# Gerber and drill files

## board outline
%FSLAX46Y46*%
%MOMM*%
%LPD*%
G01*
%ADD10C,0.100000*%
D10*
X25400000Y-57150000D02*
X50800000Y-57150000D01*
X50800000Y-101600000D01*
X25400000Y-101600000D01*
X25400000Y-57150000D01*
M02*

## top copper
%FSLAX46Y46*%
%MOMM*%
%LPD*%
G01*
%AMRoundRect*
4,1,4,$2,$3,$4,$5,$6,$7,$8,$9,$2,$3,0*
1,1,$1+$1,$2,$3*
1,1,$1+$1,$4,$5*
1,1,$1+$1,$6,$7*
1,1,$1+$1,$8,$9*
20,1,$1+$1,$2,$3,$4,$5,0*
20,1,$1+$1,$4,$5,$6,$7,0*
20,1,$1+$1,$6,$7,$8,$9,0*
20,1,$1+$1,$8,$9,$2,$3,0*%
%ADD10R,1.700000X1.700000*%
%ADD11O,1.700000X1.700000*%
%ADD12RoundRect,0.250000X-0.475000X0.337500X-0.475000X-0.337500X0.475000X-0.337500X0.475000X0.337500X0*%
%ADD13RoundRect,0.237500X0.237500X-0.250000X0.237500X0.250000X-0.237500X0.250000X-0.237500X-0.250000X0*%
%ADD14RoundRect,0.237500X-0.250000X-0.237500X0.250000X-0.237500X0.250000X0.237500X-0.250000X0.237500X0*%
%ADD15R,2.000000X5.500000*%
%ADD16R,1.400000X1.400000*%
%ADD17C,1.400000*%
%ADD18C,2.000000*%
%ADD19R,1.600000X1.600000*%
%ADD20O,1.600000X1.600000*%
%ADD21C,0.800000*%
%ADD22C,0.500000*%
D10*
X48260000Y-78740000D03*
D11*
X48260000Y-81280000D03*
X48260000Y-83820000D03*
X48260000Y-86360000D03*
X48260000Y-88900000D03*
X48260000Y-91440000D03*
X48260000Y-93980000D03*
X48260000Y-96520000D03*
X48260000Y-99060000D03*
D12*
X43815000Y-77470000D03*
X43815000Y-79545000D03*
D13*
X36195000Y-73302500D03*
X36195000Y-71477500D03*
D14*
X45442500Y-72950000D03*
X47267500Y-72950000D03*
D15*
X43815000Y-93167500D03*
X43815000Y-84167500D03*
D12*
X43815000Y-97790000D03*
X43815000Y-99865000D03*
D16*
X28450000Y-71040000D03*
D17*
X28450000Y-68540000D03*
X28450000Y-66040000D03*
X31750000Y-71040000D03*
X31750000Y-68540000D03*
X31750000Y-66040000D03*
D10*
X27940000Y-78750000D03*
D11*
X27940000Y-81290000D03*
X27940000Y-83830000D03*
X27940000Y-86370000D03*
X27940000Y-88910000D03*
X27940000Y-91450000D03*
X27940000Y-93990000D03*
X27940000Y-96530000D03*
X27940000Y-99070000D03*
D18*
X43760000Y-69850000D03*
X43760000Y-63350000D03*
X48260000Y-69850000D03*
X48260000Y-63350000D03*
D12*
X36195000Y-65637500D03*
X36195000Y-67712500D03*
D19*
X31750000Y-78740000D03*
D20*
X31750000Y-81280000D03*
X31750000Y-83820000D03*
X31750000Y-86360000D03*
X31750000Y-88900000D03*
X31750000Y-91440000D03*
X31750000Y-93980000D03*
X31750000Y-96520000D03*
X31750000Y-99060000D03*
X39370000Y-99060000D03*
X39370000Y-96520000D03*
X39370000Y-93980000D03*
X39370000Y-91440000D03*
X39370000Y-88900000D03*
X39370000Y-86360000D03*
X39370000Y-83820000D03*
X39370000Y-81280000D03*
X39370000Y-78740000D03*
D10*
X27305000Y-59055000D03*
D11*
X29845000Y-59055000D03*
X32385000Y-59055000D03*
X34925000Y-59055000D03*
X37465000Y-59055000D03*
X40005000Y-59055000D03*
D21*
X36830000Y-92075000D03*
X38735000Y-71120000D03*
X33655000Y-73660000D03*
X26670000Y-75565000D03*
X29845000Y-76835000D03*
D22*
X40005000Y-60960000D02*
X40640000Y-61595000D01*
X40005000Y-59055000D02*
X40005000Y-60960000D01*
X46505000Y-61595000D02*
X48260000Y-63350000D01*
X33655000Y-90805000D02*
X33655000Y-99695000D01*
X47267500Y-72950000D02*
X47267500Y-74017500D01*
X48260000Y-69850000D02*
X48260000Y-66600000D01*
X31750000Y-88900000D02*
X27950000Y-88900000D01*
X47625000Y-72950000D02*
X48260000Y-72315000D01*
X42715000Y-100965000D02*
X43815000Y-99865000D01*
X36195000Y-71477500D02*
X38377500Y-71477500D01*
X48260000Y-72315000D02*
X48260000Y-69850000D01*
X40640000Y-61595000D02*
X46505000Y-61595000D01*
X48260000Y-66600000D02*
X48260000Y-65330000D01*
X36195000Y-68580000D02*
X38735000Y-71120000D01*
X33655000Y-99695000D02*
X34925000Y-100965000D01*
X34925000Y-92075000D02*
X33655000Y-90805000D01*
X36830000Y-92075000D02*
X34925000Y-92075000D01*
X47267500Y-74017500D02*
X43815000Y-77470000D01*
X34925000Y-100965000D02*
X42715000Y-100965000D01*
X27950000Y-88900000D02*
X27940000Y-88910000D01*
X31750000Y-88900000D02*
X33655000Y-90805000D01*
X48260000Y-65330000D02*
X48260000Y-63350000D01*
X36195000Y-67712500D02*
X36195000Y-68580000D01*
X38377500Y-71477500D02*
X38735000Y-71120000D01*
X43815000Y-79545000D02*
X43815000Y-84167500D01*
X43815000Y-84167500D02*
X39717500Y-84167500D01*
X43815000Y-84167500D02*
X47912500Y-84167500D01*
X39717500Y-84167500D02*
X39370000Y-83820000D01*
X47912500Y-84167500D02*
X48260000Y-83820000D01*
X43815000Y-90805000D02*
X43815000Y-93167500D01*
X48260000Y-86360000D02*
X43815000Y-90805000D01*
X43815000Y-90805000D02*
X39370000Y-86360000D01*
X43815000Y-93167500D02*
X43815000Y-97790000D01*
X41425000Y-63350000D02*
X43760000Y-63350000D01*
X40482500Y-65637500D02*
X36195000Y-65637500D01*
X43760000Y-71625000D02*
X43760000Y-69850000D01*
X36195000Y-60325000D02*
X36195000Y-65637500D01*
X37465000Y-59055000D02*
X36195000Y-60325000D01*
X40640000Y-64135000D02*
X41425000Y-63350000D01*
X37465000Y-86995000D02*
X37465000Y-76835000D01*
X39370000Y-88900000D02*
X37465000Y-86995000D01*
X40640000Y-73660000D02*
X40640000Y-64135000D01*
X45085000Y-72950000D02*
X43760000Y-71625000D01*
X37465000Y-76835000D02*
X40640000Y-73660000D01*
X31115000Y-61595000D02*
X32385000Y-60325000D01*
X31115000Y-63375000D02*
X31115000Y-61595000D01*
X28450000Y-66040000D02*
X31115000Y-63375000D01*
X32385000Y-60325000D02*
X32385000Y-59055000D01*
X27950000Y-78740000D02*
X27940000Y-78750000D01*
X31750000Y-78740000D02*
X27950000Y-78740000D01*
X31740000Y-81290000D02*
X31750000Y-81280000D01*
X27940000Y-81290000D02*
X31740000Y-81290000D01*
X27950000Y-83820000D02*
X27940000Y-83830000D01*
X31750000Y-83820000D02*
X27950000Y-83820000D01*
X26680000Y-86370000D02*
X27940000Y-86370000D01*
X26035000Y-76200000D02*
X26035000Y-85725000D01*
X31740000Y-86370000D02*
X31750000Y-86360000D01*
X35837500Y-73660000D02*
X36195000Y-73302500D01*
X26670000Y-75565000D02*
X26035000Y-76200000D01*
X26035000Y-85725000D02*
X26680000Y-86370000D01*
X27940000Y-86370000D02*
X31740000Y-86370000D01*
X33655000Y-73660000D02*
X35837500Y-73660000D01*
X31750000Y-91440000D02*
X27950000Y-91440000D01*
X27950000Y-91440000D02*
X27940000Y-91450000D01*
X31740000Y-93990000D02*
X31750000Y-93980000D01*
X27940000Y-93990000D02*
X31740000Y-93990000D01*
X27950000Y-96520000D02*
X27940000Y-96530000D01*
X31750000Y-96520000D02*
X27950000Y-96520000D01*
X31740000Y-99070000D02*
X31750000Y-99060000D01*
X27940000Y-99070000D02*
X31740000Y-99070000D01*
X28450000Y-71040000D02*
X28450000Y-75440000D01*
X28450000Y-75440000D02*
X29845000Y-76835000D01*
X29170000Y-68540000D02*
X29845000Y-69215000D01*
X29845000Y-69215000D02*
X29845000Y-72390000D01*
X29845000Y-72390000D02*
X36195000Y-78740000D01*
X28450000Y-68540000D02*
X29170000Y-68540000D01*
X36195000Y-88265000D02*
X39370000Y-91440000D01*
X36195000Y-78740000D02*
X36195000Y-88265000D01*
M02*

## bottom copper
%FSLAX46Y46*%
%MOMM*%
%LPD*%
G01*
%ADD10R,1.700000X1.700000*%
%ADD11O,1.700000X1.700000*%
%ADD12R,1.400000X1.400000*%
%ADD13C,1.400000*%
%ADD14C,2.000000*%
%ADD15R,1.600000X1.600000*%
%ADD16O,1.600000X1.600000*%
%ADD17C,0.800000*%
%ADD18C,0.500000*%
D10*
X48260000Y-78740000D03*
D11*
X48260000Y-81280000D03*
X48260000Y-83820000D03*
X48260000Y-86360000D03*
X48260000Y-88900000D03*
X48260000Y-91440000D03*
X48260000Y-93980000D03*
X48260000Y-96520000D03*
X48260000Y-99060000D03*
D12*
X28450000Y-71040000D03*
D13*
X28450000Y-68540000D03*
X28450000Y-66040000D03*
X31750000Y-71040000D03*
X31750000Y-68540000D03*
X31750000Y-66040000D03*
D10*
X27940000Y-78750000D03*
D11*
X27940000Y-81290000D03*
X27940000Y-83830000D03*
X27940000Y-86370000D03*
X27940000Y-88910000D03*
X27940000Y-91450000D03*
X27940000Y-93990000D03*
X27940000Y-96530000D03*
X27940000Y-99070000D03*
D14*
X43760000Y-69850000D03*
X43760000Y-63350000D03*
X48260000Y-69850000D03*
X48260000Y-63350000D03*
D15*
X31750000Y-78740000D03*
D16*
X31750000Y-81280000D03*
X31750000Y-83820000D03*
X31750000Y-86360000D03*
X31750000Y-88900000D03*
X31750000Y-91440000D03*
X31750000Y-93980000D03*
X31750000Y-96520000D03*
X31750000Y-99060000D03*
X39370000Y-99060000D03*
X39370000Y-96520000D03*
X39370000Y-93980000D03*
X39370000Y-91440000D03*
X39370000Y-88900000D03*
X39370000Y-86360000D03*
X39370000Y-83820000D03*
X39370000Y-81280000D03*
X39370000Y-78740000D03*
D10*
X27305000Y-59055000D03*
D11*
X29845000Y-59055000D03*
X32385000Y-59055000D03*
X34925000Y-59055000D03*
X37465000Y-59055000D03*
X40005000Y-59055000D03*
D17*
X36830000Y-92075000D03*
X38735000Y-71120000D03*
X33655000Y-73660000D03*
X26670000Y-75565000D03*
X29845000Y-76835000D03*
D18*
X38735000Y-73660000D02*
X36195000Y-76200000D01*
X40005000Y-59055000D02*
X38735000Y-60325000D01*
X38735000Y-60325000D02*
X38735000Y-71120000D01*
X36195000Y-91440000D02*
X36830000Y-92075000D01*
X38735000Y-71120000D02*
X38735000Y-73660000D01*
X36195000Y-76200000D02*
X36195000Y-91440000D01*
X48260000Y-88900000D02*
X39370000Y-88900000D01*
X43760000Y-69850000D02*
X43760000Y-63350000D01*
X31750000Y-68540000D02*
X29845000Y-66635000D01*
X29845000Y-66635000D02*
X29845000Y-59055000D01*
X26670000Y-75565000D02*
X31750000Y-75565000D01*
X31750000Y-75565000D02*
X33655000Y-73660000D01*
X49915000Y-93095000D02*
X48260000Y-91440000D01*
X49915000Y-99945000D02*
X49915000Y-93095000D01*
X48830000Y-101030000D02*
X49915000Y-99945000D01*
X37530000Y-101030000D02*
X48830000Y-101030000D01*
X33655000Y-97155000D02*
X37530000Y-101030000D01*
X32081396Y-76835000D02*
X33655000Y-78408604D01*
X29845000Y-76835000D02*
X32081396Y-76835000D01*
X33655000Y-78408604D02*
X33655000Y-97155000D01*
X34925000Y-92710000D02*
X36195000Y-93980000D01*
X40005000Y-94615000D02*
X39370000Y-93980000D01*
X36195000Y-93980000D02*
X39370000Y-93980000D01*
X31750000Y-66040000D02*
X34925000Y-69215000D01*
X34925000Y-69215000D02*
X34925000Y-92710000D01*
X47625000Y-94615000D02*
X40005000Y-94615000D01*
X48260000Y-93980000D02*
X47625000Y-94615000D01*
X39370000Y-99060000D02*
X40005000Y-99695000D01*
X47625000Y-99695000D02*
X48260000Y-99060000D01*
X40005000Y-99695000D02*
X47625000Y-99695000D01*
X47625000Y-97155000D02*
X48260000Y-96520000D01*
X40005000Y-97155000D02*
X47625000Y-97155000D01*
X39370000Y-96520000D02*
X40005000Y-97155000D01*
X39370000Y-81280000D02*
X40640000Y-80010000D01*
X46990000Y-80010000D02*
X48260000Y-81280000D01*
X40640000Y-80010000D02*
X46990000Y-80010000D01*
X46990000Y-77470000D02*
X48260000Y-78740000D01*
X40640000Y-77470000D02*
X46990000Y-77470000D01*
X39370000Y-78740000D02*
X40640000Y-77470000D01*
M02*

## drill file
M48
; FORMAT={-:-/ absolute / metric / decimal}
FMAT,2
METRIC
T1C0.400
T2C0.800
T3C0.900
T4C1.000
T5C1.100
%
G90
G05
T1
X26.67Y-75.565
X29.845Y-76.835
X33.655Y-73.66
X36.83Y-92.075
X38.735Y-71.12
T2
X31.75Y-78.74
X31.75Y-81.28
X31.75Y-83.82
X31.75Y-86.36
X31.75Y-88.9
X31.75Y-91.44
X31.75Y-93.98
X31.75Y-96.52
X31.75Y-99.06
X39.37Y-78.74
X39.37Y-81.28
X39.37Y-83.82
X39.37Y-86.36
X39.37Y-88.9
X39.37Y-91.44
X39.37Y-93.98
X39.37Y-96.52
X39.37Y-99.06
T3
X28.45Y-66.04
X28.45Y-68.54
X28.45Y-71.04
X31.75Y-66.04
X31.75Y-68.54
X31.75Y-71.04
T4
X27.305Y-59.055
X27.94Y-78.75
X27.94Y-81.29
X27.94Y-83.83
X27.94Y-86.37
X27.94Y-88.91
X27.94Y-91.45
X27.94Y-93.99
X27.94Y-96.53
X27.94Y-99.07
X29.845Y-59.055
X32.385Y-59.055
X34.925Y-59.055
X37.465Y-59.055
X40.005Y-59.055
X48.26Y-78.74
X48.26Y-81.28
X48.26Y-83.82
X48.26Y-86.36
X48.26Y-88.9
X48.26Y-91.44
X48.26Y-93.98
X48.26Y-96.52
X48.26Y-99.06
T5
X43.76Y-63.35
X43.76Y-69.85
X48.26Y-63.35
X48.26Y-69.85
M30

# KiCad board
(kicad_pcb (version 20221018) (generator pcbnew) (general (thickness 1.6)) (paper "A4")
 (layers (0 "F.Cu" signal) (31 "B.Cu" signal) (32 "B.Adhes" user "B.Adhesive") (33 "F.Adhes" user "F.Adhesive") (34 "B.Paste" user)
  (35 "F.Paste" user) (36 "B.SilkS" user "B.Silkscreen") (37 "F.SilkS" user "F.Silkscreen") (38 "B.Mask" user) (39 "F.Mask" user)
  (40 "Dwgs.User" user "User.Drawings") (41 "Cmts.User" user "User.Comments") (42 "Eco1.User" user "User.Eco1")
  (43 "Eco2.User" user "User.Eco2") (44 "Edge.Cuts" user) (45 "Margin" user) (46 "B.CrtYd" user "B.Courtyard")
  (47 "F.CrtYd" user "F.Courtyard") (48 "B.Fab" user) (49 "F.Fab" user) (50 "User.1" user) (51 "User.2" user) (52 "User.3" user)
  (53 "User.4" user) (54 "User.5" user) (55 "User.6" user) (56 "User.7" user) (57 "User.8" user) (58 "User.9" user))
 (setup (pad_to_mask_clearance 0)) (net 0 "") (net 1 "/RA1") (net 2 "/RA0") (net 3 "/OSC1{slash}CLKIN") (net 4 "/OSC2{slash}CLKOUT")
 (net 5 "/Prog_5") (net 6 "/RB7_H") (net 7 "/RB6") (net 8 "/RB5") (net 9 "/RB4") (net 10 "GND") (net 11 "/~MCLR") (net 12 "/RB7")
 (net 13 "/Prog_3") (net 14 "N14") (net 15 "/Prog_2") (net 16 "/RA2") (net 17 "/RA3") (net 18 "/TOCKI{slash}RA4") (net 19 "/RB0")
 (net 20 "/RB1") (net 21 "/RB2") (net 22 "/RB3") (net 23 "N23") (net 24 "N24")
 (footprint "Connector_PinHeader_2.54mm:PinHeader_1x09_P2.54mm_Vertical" (layer "F.Cu") (at 48.26 78.74)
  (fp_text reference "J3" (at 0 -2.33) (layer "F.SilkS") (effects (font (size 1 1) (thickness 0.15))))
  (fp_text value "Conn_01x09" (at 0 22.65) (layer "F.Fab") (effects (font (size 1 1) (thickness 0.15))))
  (pad "1" thru_hole rect (at 0 0) (size 1.7 1.7) (drill 1) (layers "*.Cu" "*.Mask") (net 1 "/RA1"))
  (pad "2" thru_hole oval (at 0 2.54) (size 1.7 1.7) (drill 1) (layers "*.Cu" "*.Mask") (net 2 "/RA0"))
  (pad "3" thru_hole oval (at 0 5.08) (size 1.7 1.7) (drill 1) (layers "*.Cu" "*.Mask") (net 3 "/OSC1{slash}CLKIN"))
  (pad "4" thru_hole oval (at 0 7.62) (size 1.7 1.7) (drill 1) (layers "*.Cu" "*.Mask") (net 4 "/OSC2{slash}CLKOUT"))
  (pad "5" thru_hole oval (at 0 10.16) (size 1.7 1.7) (drill 1) (layers "*.Cu" "*.Mask") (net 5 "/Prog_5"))
  (pad "6" thru_hole oval (at 0 12.7) (size 1.7 1.7) (drill 1) (layers "*.Cu" "*.Mask") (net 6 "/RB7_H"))
  (pad "7" thru_hole oval (at 0 15.24) (size 1.7 1.7) (drill 1) (layers "*.Cu" "*.Mask") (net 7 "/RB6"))
  (pad "8" thru_hole oval (at 0 17.78) (size 1.7 1.7) (drill 1) (layers "*.Cu" "*.Mask") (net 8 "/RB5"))
  (pad "9" thru_hole oval (at 0 20.32) (size 1.7 1.7) (drill 1) (layers "*.Cu" "*.Mask") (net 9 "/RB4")))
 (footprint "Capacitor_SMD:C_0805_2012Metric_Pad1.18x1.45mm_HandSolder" (layer "F.Cu") (at 43.815 78.5075 -90)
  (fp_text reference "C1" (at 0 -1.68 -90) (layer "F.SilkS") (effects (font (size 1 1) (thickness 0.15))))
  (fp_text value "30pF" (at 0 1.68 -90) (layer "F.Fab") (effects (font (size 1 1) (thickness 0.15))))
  (pad "1" smd roundrect (at -1.0375 0 270) (size 1.175 1.45) (layers "F.Cu" "F.Paste" "F.Mask") (roundrect_rratio 0.2127659574)
   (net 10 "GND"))
  (pad "2" smd roundrect (at 1.0375 0 270) (size 1.175 1.45) (layers "F.Cu" "F.Paste" "F.Mask") (roundrect_rratio 0.2127659574)
   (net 3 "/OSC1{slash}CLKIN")))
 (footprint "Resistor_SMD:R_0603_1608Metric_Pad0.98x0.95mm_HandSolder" (layer "F.Cu") (at 36.195 72.39 90)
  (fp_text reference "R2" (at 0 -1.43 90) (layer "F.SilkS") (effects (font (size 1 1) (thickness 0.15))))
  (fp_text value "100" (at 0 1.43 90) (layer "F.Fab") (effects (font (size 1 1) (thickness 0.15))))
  (pad "1" smd roundrect (at -0.9125 0 90) (size 0.975 0.95) (layers "F.Cu" "F.Paste" "F.Mask") (roundrect_rratio 0.25) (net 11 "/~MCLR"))
  (pad "2" smd roundrect (at 0.9125 0 90) (size 0.975 0.95) (layers "F.Cu" "F.Paste" "F.Mask") (roundrect_rratio 0.25) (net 10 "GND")))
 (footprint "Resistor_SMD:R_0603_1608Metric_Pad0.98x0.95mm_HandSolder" (layer "F.Cu") (at 46.355 72.95)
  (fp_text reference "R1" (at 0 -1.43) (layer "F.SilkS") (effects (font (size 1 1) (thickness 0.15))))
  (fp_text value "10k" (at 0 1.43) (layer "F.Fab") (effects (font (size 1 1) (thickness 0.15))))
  (pad "1" smd roundrect (at -0.9125 0) (size 0.975 0.95) (layers "F.Cu" "F.Paste" "F.Mask") (roundrect_rratio 0.25) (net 5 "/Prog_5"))
  (pad "2" smd roundrect (at 0.9125 0) (size 0.975 0.95) (layers "F.Cu" "F.Paste" "F.Mask") (roundrect_rratio 0.25) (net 10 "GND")))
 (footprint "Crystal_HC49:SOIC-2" (layer "F.Cu") (at 43.815 88.6675)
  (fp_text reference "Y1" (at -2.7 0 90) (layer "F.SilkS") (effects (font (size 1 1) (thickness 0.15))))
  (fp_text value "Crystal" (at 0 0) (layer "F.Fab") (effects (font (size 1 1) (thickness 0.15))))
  (pad "1" smd rect (at 0 4.5) (size 2 5.5) (layers "F.Cu" "F.Paste" "F.Mask") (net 4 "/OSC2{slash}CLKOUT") (thermal_bridge_angle 45))
  (pad "2" smd rect (at 0 -4.5) (size 2 5.5) (layers "F.Cu" "F.Paste" "F.Mask") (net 3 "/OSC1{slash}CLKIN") (thermal_bridge_angle 45)))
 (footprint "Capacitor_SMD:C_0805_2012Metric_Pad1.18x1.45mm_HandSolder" (layer "F.Cu") (at 43.815 98.8275 -90)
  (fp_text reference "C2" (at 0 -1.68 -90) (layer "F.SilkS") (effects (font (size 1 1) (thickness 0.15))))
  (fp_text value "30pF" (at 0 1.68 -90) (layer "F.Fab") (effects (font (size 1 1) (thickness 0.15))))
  (pad "1" smd roundrect (at -1.0375 0 270) (size 1.175 1.45) (layers "F.Cu" "F.Paste" "F.Mask") (roundrect_rratio 0.2127659574)
   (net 4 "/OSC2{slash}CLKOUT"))
  (pad "2" smd roundrect (at 1.0375 0 270) (size 1.175 1.45) (layers "F.Cu" "F.Paste" "F.Mask") (roundrect_rratio 0.2127659574)
   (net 10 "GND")))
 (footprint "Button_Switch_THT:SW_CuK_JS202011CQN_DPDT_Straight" (layer "F.Cu") (at 28.45 71.04 90)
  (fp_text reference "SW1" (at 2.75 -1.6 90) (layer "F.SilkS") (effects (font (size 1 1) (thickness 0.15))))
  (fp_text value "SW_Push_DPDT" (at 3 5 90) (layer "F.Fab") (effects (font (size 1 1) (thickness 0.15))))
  (pad "1" thru_hole rect (at 0 0 90) (size 1.4 1.4) (drill 0.9) (layers "*.Cu" "*.Mask") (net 6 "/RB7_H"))
  (pad "2" thru_hole circle (at 2.5 0 90) (size 1.4 1.4) (drill 0.9) (layers "*.Cu" "*.Mask") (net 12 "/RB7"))
  (pad "3" thru_hole circle (at 5 0 90) (size 1.4 1.4) (drill 0.9) (layers "*.Cu" "*.Mask") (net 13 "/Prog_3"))
  (pad "4" thru_hole circle (at 0 3.3 90) (size 1.4 1.4) (drill 0.9) (layers "*.Cu" "*.Mask") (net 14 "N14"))
  (pad "5" thru_hole circle (at 2.5 3.3 90) (size 1.4 1.4) (drill 0.9) (layers "*.Cu" "*.Mask") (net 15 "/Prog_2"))
  (pad "6" thru_hole circle (at 5 3.3 90) (size 1.4 1.4) (drill 0.9) (layers "*.Cu" "*.Mask") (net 7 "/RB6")))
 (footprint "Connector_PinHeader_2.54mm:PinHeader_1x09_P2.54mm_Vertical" (layer "F.Cu") (at 27.94 78.75)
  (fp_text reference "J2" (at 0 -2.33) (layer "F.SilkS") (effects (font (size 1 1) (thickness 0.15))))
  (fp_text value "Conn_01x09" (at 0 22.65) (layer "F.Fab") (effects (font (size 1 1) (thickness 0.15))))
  (pad "1" thru_hole rect (at 0 0) (size 1.7 1.7) (drill 1) (layers "*.Cu" "*.Mask") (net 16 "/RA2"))
  (pad "2" thru_hole oval (at 0 2.54) (size 1.7 1.7) (drill 1) (layers "*.Cu" "*.Mask") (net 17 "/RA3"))
  (pad "3" thru_hole oval (at 0 5.08) (size 1.7 1.7) (drill 1) (layers "*.Cu" "*.Mask") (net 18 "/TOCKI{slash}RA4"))
  (pad "4" thru_hole oval (at 0 7.62) (size 1.7 1.7) (drill 1) (layers "*.Cu" "*.Mask") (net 11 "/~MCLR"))
  (pad "5" thru_hole oval (at 0 10.16) (size 1.7 1.7) (drill 1) (layers "*.Cu" "*.Mask") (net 10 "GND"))
  (pad "6" thru_hole oval (at 0 12.7) (size 1.7 1.7) (drill 1) (layers "*.Cu" "*.Mask") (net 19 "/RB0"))
  (pad "7" thru_hole oval (at 0 15.24) (size 1.7 1.7) (drill 1) (layers "*.Cu" "*.Mask") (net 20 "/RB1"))
  (pad "8" thru_hole oval (at 0 17.78) (size 1.7 1.7) (drill 1) (layers "*.Cu" "*.Mask") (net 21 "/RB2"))
  (pad "9" thru_hole oval (at 0 20.32) (size 1.7 1.7) (drill 1) (layers "*.Cu" "*.Mask") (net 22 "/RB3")))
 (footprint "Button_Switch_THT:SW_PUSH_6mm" (layer "F.Cu") (at 43.76 69.85 90)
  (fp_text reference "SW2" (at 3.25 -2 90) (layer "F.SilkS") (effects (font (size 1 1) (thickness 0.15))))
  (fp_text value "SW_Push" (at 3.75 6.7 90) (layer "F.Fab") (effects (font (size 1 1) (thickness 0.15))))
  (pad "1" thru_hole circle (at 0 0 180) (size 2 2) (drill 1.1) (layers "*.Cu" "*.Mask") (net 5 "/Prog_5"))
  (pad "1" thru_hole circle (at 6.5 0 180) (size 2 2) (drill 1.1) (layers "*.Cu" "*.Mask") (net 5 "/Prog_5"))
  (pad "2" thru_hole circle (at 0 4.5 180) (size 2 2) (drill 1.1) (layers "*.Cu" "*.Mask") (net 10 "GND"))
  (pad "2" thru_hole circle (at 6.5 4.5 180) (size 2 2) (drill 1.1) (layers "*.Cu" "*.Mask") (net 10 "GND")))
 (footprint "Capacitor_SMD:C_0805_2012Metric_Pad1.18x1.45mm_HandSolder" (layer "F.Cu") (at 36.195 66.675 -90)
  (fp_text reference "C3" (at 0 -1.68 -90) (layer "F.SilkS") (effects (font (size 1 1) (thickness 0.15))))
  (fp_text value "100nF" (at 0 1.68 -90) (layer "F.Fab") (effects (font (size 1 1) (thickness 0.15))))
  (pad "1" smd roundrect (at -1.0375 0 270) (size 1.175 1.45) (layers "F.Cu" "F.Paste" "F.Mask") (roundrect_rratio 0.2127659574)
   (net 5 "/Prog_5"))
  (pad "2" smd roundrect (at 1.0375 0 270) (size 1.175 1.45) (layers "F.Cu" "F.Paste" "F.Mask") (roundrect_rratio 0.2127659574)
   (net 10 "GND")))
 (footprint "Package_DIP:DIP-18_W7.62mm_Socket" (layer "F.Cu") (at 31.75 78.74)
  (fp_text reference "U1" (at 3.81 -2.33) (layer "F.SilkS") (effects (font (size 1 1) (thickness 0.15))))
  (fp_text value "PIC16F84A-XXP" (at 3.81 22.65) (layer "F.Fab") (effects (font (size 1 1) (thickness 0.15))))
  (pad "1" thru_hole rect (at 0 0) (size 1.6 1.6) (drill 0.8) (layers "*.Cu" "*.Mask") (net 16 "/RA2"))
  (pad "2" thru_hole oval (at 0 2.54) (size 1.6 1.6) (drill 0.8) (layers "*.Cu" "*.Mask") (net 17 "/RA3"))
  (pad "3" thru_hole oval (at 0 5.08) (size 1.6 1.6) (drill 0.8) (layers "*.Cu" "*.Mask") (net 18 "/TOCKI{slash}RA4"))
  (pad "4" thru_hole oval (at 0 7.62) (size 1.6 1.6) (drill 0.8) (layers "*.Cu" "*.Mask") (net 11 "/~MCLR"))
  (pad "5" thru_hole oval (at 0 10.16) (size 1.6 1.6) (drill 0.8) (layers "*.Cu" "*.Mask") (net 10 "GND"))
  (pad "6" thru_hole oval (at 0 12.7) (size 1.6 1.6) (drill 0.8) (layers "*.Cu" "*.Mask") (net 19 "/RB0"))
  (pad "7" thru_hole oval (at 0 15.24) (size 1.6 1.6) (drill 0.8) (layers "*.Cu" "*.Mask") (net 20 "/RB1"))
  (pad "8" thru_hole oval (at 0 17.78) (size 1.6 1.6) (drill 0.8) (layers "*.Cu" "*.Mask") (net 21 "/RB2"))
  (pad "9" thru_hole oval (at 0 20.32) (size 1.6 1.6) (drill 0.8) (layers "*.Cu" "*.Mask") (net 22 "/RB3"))
  (pad "10" thru_hole oval (at 7.62 20.32) (size 1.6 1.6) (drill 0.8) (layers "*.Cu" "*.Mask") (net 9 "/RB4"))
  (pad "11" thru_hole oval (at 7.62 17.78) (size 1.6 1.6) (drill 0.8) (layers "*.Cu" "*.Mask") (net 8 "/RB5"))
  (pad "12" thru_hole oval (at 7.62 15.24) (size 1.6 1.6) (drill 0.8) (layers "*.Cu" "*.Mask") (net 7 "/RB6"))
  (pad "13" thru_hole oval (at 7.62 12.7) (size 1.6 1.6) (drill 0.8) (layers "*.Cu" "*.Mask") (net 12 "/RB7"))
  (pad "14" thru_hole oval (at 7.62 10.16) (size 1.6 1.6) (drill 0.8) (layers "*.Cu" "*.Mask") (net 5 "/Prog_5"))
  (pad "15" thru_hole oval (at 7.62 7.62) (size 1.6 1.6) (drill 0.8) (layers "*.Cu" "*.Mask") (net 4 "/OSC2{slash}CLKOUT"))
  (pad "16" thru_hole oval (at 7.62 5.08) (size 1.6 1.6) (drill 0.8) (layers "*.Cu" "*.Mask") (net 3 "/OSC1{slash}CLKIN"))
  (pad "17" thru_hole oval (at 7.62 2.54) (size 1.6 1.6) (drill 0.8) (layers "*.Cu" "*.Mask") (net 2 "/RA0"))
  (pad "18" thru_hole oval (at 7.62 0) (size 1.6 1.6) (drill 0.8) (layers "*.Cu" "*.Mask") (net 1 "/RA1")))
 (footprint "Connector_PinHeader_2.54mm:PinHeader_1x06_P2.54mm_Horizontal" (layer "F.Cu") (at 27.305 59.055 90)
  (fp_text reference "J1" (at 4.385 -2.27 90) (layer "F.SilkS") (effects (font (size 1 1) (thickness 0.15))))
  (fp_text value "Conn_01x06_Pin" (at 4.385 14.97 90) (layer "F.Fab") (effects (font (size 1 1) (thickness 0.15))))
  (pad "1" thru_hole rect (at 0 0 90) (size 1.7 1.7) (drill 1) (layers "*.Cu" "*.Mask") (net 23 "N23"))
  (pad "2" thru_hole oval (at 0 2.54 90) (size 1.7 1.7) (drill 1) (layers "*.Cu" "*.Mask") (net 15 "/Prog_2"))
  (pad "3" thru_hole oval (at 0 5.08 90) (size 1.7 1.7) (drill 1) (layers "*.Cu" "*.Mask") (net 13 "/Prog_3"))
  (pad "4" thru_hole oval (at 0 7.62 90) (size 1.7 1.7) (drill 1) (layers "*.Cu" "*.Mask") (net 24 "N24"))
  (pad "5" thru_hole oval (at 0 10.16 90) (size 1.7 1.7) (drill 1) (layers "*.Cu" "*.Mask") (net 5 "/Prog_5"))
  (pad "6" thru_hole oval (at 0 12.7 90) (size 1.7 1.7) (drill 1) (layers "*.Cu" "*.Mask") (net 10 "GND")))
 (gr_rect (start 25.4 57.15) (end 50.8 101.6) (stroke (width 0.1) (type default)) (fill none) (layer "Edge.Cuts"))
 (segment (start 40.005 60.96) (end 40.64 61.595) (width 0.5) (layer "F.Cu") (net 10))
 (segment (start 40.005 59.055) (end 40.005 60.96) (width 0.5) (layer "F.Cu") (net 10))
 (segment (start 46.505 61.595) (end 48.26 63.35) (width 0.5) (layer "F.Cu") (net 10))
 (segment (start 33.655 90.805) (end 33.655 99.695) (width 0.5) (layer "F.Cu") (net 10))
 (segment (start 47.2675 72.95) (end 47.2675 74.0175) (width 0.5) (layer "F.Cu") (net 10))
 (segment (start 48.26 69.85) (end 48.26 66.6) (width 0.5) (layer "F.Cu") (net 10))
 (segment (start 31.75 88.9) (end 27.95 88.9) (width 0.5) (layer "F.Cu") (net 10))
 (segment (start 47.625 72.95) (end 48.26 72.315) (width 0.5) (layer "F.Cu") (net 10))
 (segment (start 42.715 100.965) (end 43.815 99.865) (width 0.5) (layer "F.Cu") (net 10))
 (segment (start 36.195 71.4775) (end 38.3775 71.4775) (width 0.5) (layer "F.Cu") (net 10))
 (segment (start 48.26 72.315) (end 48.26 69.85) (width 0.5) (layer "F.Cu") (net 10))
 (segment (start 40.64 61.595) (end 46.505 61.595) (width 0.5) (layer "F.Cu") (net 10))
 (segment (start 48.26 66.6) (end 48.26 65.33) (width 0.5) (layer "F.Cu") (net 10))
 (segment (start 36.195 68.58) (end 38.735 71.12) (width 0.5) (layer "F.Cu") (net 10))
 (segment (start 33.655 99.695) (end 34.925 100.965) (width 0.5) (layer "F.Cu") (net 10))
 (segment (start 34.925 92.075) (end 33.655 90.805) (width 0.5) (layer "F.Cu") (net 10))
 (segment (start 36.83 92.075) (end 34.925 92.075) (width 0.5) (layer "F.Cu") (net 10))
 (segment (start 47.2675 74.0175) (end 43.815 77.47) (width 0.5) (layer "F.Cu") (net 10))
 (segment (start 34.925 100.965) (end 42.715 100.965) (width 0.5) (layer "F.Cu") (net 10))
 (segment (start 27.95 88.9) (end 27.94 88.91) (width 0.5) (layer "F.Cu") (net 10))
 (segment (start 31.75 88.9) (end 33.655 90.805) (width 0.5) (layer "F.Cu") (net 10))
 (segment (start 48.26 65.33) (end 48.26 63.35) (width 0.5) (layer "F.Cu") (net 10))
 (segment (start 36.195 67.7125) (end 36.195 68.58) (width 0.5) (layer "F.Cu") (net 10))
 (segment (start 38.3775 71.4775) (end 38.735 71.12) (width 0.5) (layer "F.Cu") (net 10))
 (via (at 36.83 92.075) (size 0.8) (drill 0.4) (layers "F.Cu" "B.Cu") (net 10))
 (via (at 38.735 71.12) (size 0.8) (drill 0.4) (layers "F.Cu" "B.Cu") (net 10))
 (segment (start 38.735 73.66) (end 36.195 76.2) (width 0.5) (layer "B.Cu") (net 10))
 (segment (start 40.005 59.055) (end 38.735 60.325) (width 0.5) (layer "B.Cu") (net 10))
 (segment (start 38.735 60.325) (end 38.735 71.12) (width 0.5) (layer "B.Cu") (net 10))
 (segment (start 36.195 91.44) (end 36.83 92.075) (width 0.5) (layer "B.Cu") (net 10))
 (segment (start 38.735 71.12) (end 38.735 73.66) (width 0.5) (layer "B.Cu") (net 10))
 (segment (start 36.195 76.2) (end 36.195 91.44) (width 0.5) (layer "B.Cu") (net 10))
 (segment (start 43.815 79.545) (end 43.815 84.1675) (width 0.5) (layer "F.Cu") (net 3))
 (segment (start 43.815 84.1675) (end 39.7175 84.1675) (width 0.5) (layer "F.Cu") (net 3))
 (segment (start 43.815 84.1675) (end 47.9125 84.1675) (width 0.5) (layer "F.Cu") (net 3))
 (segment (start 39.7175 84.1675) (end 39.37 83.82) (width 0.5) (layer "F.Cu") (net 3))
 (segment (start 47.9125 84.1675) (end 48.26 83.82) (width 0.5) (layer "F.Cu") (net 3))
 (segment (start 43.815 90.805) (end 43.815 93.1675) (width 0.5) (layer "F.Cu") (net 4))
 (segment (start 48.26 86.36) (end 43.815 90.805) (width 0.5) (layer "F.Cu") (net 4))
 (segment (start 43.815 90.805) (end 39.37 86.36) (width 0.5) (layer "F.Cu") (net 4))
 (segment (start 43.815 93.1675) (end 43.815 97.79) (width 0.5) (layer "F.Cu") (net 4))
 (segment (start 41.425 63.35) (end 43.76 63.35) (width 0.5) (layer "F.Cu") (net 5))
 (segment (start 40.4825 65.6375) (end 36.195 65.6375) (width 0.5) (layer "F.Cu") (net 5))
 (segment (start 43.76 71.625) (end 43.76 69.85) (width 0.5) (layer "F.Cu") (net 5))
 (segment (start 36.195 60.325) (end 36.195 65.6375) (width 0.5) (layer "F.Cu") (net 5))
 (segment (start 37.465 59.055) (end 36.195 60.325) (width 0.5) (layer "F.Cu") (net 5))
 (segment (start 40.64 64.135) (end 41.425 63.35) (width 0.5) (layer "F.Cu") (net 5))
 (segment (start 37.465 86.995) (end 37.465 76.835) (width 0.5) (layer "F.Cu") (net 5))
 (segment (start 39.37 88.9) (end 37.465 86.995) (width 0.5) (layer "F.Cu") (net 5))
 (segment (start 40.64 73.66) (end 40.64 64.135) (width 0.5) (layer "F.Cu") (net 5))
 (segment (start 45.085 72.95) (end 43.76 71.625) (width 0.5) (layer "F.Cu") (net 5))
 (segment (start 37.465 76.835) (end 40.64 73.66) (width 0.5) (layer "F.Cu") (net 5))
 (segment (start 48.26 88.9) (end 39.37 88.9) (width 0.5) (layer "B.Cu") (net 5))
 (segment (start 43.76 69.85) (end 43.76 63.35) (width 0.5) (layer "B.Cu") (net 5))
 (segment (start 31.75 68.54) (end 29.845 66.635) (width 0.5) (layer "B.Cu") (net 15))
 (segment (start 29.845 66.635) (end 29.845 59.055) (width 0.5) (layer "B.Cu") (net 15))
 (segment (start 31.115 61.595) (end 32.385 60.325) (width 0.5) (layer "F.Cu") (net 13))
 (segment (start 31.115 63.375) (end 31.115 61.595) (width 0.5) (layer "F.Cu") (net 13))
 (segment (start 28.45 66.04) (end 31.115 63.375) (width 0.5) (layer "F.Cu") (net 13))
 (segment (start 32.385 60.325) (end 32.385 59.055) (width 0.5) (layer "F.Cu") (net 13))
 (segment (start 27.95 78.74) (end 27.94 78.75) (width 0.5) (layer "F.Cu") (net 16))
 (segment (start 31.75 78.74) (end 27.95 78.74) (width 0.5) (layer "F.Cu") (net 16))
 (segment (start 31.74 81.29) (end 31.75 81.28) (width 0.5) (layer "F.Cu") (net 17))
 (segment (start 27.94 81.29) (end 31.74 81.29) (width 0.5) (layer "F.Cu") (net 17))
 (segment (start 27.95 83.82) (end 27.94 83.83) (width 0.5) (layer "F.Cu") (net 18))
 (segment (start 31.75 83.82) (end 27.95 83.82) (width 0.5) (layer "F.Cu") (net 18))
 (segment (start 26.68 86.37) (end 27.94 86.37) (width 0.5) (layer "F.Cu") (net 11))
 (segment (start 26.035 76.2) (end 26.035 85.725) (width 0.5) (layer "F.Cu") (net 11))
 (segment (start 31.74 86.37) (end 31.75 86.36) (width 0.5) (layer "F.Cu") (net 11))
 (segment (start 35.8375 73.66) (end 36.195 73.3025) (width 0.5) (layer "F.Cu") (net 11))
 (segment (start 26.67 75.565) (end 26.035 76.2) (width 0.5) (layer "F.Cu") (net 11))
 (segment (start 26.035 85.725) (end 26.68 86.37) (width 0.5) (layer "F.Cu") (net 11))
 (segment (start 27.94 86.37) (end 31.74 86.37) (width 0.5) (layer "F.Cu") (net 11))
 (segment (start 33.655 73.66) (end 35.8375 73.66) (width 0.5) (layer "F.Cu") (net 11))
 (via (at 33.655 73.66) (size 0.8) (drill 0.4) (layers "F.Cu" "B.Cu") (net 11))
 (via (at 26.67 75.565) (size 0.8) (drill 0.4) (layers "F.Cu" "B.Cu") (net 11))
 (segment (start 26.67 75.565) (end 31.75 75.565) (width 0.5) (layer "B.Cu") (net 11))
 (segment (start 31.75 75.565) (end 33.655 73.66) (width 0.5) (layer "B.Cu") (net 11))
 (segment (start 31.75 91.44) (end 27.95 91.44) (width 0.5) (layer "F.Cu") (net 19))
 (segment (start 27.95 91.44) (end 27.94 91.45) (width 0.5) (layer "F.Cu") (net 19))
 (segment (start 31.74 93.99) (end 31.75 93.98) (width 0.5) (layer "F.Cu") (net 20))
 (segment (start 27.94 93.99) (end 31.74 93.99) (width 0.5) (layer "F.Cu") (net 20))
 (segment (start 27.95 96.52) (end 27.94 96.53) (width 0.5) (layer "F.Cu") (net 21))
 (segment (start 31.75 96.52) (end 27.95 96.52) (width 0.5) (layer "F.Cu") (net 21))
 (segment (start 31.74 99.07) (end 31.75 99.06) (width 0.5) (layer "F.Cu") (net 22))
 (segment (start 27.94 99.07) (end 31.74 99.07) (width 0.5) (layer "F.Cu") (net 22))
 (segment (start 28.45 71.04) (end 28.45 75.44) (width 0.5) (layer "F.Cu") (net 6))
 (segment (start 28.45 75.44) (end 29.845 76.835) (width 0.5) (layer "F.Cu") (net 6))
 (via (at 29.845 76.835) (size 0.8) (drill 0.4) (layers "F.Cu" "B.Cu") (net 6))
 (segment (start 49.915 93.095) (end 48.26 91.44) (width 0.5) (layer "B.Cu") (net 6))
 (segment (start 49.915 99.945) (end 49.915 93.095) (width 0.5) (layer "B.Cu") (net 6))
 (segment (start 48.83 101.03) (end 49.915 99.945) (width 0.5) (layer "B.Cu") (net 6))
 (segment (start 37.53 101.03) (end 48.83 101.03) (width 0.5) (layer "B.Cu") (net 6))
 (segment (start 33.655 97.155) (end 37.53 101.03) (width 0.5) (layer "B.Cu") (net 6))
 (segment (start 32.081396 76.835) (end 33.655 78.408604) (width 0.5) (layer "B.Cu") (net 6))
 (segment (start 29.845 76.835) (end 32.081396 76.835) (width 0.5) (layer "B.Cu") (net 6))
 (segment (start 33.655 78.408604) (end 33.655 97.155) (width 0.5) (layer "B.Cu") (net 6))
 (segment (start 29.17 68.54) (end 29.845 69.215) (width 0.5) (layer "F.Cu") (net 12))
 (segment (start 29.845 69.215) (end 29.845 72.39) (width 0.5) (layer "F.Cu") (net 12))
 (segment (start 29.845 72.39) (end 36.195 78.74) (width 0.5) (layer "F.Cu") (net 12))
 (segment (start 28.45 68.54) (end 29.17 68.54) (width 0.5) (layer "F.Cu") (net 12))
 (segment (start 36.195 88.265) (end 39.37 91.44) (width 0.5) (layer "F.Cu") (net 12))
 (segment (start 36.195 78.74) (end 36.195 88.265) (width 0.5) (layer "F.Cu") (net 12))
 (segment (start 34.925 92.71) (end 36.195 93.98) (width 0.5) (layer "B.Cu") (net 7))
 (segment (start 40.005 94.615) (end 39.37 93.98) (width 0.5) (layer "B.Cu") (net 7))
 (segment (start 36.195 93.98) (end 39.37 93.98) (width 0.5) (layer "B.Cu") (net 7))
 (segment (start 31.75 66.04) (end 34.925 69.215) (width 0.5) (layer "B.Cu") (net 7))
 (segment (start 34.925 69.215) (end 34.925 92.71) (width 0.5) (layer "B.Cu") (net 7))
 (segment (start 47.625 94.615) (end 40.005 94.615) (width 0.5) (layer "B.Cu") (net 7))
 (segment (start 48.26 93.98) (end 47.625 94.615) (width 0.5) (layer "B.Cu") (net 7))
 (segment (start 39.37 99.06) (end 40.005 99.695) (width 0.5) (layer "B.Cu") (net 9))
 (segment (start 47.625 99.695) (end 48.26 99.06) (width 0.5) (layer "B.Cu") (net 9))
 (segment (start 40.005 99.695) (end 47.625 99.695) (width 0.5) (layer "B.Cu") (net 9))
 (segment (start 47.625 97.155) (end 48.26 96.52) (width 0.5) (layer "B.Cu") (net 8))
 (segment (start 40.005 97.155) (end 47.625 97.155) (width 0.5) (layer "B.Cu") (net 8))
 (segment (start 39.37 96.52) (end 40.005 97.155) (width 0.5) (layer "B.Cu") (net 8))
 (segment (start 39.37 81.28) (end 40.64 80.01) (width 0.5) (layer "B.Cu") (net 2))
 (segment (start 46.99 80.01) (end 48.26 81.28) (width 0.5) (layer "B.Cu") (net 2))
 (segment (start 40.64 80.01) (end 46.99 80.01) (width 0.5) (layer "B.Cu") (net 2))
 (segment (start 46.99 77.47) (end 48.26 78.74) (width 0.5) (layer "B.Cu") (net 1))
 (segment (start 40.64 77.47) (end 46.99 77.47) (width 0.5) (layer "B.Cu") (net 1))
 (segment (start 39.37 78.74) (end 40.64 77.47) (width 0.5) (layer "B.Cu") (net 1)))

